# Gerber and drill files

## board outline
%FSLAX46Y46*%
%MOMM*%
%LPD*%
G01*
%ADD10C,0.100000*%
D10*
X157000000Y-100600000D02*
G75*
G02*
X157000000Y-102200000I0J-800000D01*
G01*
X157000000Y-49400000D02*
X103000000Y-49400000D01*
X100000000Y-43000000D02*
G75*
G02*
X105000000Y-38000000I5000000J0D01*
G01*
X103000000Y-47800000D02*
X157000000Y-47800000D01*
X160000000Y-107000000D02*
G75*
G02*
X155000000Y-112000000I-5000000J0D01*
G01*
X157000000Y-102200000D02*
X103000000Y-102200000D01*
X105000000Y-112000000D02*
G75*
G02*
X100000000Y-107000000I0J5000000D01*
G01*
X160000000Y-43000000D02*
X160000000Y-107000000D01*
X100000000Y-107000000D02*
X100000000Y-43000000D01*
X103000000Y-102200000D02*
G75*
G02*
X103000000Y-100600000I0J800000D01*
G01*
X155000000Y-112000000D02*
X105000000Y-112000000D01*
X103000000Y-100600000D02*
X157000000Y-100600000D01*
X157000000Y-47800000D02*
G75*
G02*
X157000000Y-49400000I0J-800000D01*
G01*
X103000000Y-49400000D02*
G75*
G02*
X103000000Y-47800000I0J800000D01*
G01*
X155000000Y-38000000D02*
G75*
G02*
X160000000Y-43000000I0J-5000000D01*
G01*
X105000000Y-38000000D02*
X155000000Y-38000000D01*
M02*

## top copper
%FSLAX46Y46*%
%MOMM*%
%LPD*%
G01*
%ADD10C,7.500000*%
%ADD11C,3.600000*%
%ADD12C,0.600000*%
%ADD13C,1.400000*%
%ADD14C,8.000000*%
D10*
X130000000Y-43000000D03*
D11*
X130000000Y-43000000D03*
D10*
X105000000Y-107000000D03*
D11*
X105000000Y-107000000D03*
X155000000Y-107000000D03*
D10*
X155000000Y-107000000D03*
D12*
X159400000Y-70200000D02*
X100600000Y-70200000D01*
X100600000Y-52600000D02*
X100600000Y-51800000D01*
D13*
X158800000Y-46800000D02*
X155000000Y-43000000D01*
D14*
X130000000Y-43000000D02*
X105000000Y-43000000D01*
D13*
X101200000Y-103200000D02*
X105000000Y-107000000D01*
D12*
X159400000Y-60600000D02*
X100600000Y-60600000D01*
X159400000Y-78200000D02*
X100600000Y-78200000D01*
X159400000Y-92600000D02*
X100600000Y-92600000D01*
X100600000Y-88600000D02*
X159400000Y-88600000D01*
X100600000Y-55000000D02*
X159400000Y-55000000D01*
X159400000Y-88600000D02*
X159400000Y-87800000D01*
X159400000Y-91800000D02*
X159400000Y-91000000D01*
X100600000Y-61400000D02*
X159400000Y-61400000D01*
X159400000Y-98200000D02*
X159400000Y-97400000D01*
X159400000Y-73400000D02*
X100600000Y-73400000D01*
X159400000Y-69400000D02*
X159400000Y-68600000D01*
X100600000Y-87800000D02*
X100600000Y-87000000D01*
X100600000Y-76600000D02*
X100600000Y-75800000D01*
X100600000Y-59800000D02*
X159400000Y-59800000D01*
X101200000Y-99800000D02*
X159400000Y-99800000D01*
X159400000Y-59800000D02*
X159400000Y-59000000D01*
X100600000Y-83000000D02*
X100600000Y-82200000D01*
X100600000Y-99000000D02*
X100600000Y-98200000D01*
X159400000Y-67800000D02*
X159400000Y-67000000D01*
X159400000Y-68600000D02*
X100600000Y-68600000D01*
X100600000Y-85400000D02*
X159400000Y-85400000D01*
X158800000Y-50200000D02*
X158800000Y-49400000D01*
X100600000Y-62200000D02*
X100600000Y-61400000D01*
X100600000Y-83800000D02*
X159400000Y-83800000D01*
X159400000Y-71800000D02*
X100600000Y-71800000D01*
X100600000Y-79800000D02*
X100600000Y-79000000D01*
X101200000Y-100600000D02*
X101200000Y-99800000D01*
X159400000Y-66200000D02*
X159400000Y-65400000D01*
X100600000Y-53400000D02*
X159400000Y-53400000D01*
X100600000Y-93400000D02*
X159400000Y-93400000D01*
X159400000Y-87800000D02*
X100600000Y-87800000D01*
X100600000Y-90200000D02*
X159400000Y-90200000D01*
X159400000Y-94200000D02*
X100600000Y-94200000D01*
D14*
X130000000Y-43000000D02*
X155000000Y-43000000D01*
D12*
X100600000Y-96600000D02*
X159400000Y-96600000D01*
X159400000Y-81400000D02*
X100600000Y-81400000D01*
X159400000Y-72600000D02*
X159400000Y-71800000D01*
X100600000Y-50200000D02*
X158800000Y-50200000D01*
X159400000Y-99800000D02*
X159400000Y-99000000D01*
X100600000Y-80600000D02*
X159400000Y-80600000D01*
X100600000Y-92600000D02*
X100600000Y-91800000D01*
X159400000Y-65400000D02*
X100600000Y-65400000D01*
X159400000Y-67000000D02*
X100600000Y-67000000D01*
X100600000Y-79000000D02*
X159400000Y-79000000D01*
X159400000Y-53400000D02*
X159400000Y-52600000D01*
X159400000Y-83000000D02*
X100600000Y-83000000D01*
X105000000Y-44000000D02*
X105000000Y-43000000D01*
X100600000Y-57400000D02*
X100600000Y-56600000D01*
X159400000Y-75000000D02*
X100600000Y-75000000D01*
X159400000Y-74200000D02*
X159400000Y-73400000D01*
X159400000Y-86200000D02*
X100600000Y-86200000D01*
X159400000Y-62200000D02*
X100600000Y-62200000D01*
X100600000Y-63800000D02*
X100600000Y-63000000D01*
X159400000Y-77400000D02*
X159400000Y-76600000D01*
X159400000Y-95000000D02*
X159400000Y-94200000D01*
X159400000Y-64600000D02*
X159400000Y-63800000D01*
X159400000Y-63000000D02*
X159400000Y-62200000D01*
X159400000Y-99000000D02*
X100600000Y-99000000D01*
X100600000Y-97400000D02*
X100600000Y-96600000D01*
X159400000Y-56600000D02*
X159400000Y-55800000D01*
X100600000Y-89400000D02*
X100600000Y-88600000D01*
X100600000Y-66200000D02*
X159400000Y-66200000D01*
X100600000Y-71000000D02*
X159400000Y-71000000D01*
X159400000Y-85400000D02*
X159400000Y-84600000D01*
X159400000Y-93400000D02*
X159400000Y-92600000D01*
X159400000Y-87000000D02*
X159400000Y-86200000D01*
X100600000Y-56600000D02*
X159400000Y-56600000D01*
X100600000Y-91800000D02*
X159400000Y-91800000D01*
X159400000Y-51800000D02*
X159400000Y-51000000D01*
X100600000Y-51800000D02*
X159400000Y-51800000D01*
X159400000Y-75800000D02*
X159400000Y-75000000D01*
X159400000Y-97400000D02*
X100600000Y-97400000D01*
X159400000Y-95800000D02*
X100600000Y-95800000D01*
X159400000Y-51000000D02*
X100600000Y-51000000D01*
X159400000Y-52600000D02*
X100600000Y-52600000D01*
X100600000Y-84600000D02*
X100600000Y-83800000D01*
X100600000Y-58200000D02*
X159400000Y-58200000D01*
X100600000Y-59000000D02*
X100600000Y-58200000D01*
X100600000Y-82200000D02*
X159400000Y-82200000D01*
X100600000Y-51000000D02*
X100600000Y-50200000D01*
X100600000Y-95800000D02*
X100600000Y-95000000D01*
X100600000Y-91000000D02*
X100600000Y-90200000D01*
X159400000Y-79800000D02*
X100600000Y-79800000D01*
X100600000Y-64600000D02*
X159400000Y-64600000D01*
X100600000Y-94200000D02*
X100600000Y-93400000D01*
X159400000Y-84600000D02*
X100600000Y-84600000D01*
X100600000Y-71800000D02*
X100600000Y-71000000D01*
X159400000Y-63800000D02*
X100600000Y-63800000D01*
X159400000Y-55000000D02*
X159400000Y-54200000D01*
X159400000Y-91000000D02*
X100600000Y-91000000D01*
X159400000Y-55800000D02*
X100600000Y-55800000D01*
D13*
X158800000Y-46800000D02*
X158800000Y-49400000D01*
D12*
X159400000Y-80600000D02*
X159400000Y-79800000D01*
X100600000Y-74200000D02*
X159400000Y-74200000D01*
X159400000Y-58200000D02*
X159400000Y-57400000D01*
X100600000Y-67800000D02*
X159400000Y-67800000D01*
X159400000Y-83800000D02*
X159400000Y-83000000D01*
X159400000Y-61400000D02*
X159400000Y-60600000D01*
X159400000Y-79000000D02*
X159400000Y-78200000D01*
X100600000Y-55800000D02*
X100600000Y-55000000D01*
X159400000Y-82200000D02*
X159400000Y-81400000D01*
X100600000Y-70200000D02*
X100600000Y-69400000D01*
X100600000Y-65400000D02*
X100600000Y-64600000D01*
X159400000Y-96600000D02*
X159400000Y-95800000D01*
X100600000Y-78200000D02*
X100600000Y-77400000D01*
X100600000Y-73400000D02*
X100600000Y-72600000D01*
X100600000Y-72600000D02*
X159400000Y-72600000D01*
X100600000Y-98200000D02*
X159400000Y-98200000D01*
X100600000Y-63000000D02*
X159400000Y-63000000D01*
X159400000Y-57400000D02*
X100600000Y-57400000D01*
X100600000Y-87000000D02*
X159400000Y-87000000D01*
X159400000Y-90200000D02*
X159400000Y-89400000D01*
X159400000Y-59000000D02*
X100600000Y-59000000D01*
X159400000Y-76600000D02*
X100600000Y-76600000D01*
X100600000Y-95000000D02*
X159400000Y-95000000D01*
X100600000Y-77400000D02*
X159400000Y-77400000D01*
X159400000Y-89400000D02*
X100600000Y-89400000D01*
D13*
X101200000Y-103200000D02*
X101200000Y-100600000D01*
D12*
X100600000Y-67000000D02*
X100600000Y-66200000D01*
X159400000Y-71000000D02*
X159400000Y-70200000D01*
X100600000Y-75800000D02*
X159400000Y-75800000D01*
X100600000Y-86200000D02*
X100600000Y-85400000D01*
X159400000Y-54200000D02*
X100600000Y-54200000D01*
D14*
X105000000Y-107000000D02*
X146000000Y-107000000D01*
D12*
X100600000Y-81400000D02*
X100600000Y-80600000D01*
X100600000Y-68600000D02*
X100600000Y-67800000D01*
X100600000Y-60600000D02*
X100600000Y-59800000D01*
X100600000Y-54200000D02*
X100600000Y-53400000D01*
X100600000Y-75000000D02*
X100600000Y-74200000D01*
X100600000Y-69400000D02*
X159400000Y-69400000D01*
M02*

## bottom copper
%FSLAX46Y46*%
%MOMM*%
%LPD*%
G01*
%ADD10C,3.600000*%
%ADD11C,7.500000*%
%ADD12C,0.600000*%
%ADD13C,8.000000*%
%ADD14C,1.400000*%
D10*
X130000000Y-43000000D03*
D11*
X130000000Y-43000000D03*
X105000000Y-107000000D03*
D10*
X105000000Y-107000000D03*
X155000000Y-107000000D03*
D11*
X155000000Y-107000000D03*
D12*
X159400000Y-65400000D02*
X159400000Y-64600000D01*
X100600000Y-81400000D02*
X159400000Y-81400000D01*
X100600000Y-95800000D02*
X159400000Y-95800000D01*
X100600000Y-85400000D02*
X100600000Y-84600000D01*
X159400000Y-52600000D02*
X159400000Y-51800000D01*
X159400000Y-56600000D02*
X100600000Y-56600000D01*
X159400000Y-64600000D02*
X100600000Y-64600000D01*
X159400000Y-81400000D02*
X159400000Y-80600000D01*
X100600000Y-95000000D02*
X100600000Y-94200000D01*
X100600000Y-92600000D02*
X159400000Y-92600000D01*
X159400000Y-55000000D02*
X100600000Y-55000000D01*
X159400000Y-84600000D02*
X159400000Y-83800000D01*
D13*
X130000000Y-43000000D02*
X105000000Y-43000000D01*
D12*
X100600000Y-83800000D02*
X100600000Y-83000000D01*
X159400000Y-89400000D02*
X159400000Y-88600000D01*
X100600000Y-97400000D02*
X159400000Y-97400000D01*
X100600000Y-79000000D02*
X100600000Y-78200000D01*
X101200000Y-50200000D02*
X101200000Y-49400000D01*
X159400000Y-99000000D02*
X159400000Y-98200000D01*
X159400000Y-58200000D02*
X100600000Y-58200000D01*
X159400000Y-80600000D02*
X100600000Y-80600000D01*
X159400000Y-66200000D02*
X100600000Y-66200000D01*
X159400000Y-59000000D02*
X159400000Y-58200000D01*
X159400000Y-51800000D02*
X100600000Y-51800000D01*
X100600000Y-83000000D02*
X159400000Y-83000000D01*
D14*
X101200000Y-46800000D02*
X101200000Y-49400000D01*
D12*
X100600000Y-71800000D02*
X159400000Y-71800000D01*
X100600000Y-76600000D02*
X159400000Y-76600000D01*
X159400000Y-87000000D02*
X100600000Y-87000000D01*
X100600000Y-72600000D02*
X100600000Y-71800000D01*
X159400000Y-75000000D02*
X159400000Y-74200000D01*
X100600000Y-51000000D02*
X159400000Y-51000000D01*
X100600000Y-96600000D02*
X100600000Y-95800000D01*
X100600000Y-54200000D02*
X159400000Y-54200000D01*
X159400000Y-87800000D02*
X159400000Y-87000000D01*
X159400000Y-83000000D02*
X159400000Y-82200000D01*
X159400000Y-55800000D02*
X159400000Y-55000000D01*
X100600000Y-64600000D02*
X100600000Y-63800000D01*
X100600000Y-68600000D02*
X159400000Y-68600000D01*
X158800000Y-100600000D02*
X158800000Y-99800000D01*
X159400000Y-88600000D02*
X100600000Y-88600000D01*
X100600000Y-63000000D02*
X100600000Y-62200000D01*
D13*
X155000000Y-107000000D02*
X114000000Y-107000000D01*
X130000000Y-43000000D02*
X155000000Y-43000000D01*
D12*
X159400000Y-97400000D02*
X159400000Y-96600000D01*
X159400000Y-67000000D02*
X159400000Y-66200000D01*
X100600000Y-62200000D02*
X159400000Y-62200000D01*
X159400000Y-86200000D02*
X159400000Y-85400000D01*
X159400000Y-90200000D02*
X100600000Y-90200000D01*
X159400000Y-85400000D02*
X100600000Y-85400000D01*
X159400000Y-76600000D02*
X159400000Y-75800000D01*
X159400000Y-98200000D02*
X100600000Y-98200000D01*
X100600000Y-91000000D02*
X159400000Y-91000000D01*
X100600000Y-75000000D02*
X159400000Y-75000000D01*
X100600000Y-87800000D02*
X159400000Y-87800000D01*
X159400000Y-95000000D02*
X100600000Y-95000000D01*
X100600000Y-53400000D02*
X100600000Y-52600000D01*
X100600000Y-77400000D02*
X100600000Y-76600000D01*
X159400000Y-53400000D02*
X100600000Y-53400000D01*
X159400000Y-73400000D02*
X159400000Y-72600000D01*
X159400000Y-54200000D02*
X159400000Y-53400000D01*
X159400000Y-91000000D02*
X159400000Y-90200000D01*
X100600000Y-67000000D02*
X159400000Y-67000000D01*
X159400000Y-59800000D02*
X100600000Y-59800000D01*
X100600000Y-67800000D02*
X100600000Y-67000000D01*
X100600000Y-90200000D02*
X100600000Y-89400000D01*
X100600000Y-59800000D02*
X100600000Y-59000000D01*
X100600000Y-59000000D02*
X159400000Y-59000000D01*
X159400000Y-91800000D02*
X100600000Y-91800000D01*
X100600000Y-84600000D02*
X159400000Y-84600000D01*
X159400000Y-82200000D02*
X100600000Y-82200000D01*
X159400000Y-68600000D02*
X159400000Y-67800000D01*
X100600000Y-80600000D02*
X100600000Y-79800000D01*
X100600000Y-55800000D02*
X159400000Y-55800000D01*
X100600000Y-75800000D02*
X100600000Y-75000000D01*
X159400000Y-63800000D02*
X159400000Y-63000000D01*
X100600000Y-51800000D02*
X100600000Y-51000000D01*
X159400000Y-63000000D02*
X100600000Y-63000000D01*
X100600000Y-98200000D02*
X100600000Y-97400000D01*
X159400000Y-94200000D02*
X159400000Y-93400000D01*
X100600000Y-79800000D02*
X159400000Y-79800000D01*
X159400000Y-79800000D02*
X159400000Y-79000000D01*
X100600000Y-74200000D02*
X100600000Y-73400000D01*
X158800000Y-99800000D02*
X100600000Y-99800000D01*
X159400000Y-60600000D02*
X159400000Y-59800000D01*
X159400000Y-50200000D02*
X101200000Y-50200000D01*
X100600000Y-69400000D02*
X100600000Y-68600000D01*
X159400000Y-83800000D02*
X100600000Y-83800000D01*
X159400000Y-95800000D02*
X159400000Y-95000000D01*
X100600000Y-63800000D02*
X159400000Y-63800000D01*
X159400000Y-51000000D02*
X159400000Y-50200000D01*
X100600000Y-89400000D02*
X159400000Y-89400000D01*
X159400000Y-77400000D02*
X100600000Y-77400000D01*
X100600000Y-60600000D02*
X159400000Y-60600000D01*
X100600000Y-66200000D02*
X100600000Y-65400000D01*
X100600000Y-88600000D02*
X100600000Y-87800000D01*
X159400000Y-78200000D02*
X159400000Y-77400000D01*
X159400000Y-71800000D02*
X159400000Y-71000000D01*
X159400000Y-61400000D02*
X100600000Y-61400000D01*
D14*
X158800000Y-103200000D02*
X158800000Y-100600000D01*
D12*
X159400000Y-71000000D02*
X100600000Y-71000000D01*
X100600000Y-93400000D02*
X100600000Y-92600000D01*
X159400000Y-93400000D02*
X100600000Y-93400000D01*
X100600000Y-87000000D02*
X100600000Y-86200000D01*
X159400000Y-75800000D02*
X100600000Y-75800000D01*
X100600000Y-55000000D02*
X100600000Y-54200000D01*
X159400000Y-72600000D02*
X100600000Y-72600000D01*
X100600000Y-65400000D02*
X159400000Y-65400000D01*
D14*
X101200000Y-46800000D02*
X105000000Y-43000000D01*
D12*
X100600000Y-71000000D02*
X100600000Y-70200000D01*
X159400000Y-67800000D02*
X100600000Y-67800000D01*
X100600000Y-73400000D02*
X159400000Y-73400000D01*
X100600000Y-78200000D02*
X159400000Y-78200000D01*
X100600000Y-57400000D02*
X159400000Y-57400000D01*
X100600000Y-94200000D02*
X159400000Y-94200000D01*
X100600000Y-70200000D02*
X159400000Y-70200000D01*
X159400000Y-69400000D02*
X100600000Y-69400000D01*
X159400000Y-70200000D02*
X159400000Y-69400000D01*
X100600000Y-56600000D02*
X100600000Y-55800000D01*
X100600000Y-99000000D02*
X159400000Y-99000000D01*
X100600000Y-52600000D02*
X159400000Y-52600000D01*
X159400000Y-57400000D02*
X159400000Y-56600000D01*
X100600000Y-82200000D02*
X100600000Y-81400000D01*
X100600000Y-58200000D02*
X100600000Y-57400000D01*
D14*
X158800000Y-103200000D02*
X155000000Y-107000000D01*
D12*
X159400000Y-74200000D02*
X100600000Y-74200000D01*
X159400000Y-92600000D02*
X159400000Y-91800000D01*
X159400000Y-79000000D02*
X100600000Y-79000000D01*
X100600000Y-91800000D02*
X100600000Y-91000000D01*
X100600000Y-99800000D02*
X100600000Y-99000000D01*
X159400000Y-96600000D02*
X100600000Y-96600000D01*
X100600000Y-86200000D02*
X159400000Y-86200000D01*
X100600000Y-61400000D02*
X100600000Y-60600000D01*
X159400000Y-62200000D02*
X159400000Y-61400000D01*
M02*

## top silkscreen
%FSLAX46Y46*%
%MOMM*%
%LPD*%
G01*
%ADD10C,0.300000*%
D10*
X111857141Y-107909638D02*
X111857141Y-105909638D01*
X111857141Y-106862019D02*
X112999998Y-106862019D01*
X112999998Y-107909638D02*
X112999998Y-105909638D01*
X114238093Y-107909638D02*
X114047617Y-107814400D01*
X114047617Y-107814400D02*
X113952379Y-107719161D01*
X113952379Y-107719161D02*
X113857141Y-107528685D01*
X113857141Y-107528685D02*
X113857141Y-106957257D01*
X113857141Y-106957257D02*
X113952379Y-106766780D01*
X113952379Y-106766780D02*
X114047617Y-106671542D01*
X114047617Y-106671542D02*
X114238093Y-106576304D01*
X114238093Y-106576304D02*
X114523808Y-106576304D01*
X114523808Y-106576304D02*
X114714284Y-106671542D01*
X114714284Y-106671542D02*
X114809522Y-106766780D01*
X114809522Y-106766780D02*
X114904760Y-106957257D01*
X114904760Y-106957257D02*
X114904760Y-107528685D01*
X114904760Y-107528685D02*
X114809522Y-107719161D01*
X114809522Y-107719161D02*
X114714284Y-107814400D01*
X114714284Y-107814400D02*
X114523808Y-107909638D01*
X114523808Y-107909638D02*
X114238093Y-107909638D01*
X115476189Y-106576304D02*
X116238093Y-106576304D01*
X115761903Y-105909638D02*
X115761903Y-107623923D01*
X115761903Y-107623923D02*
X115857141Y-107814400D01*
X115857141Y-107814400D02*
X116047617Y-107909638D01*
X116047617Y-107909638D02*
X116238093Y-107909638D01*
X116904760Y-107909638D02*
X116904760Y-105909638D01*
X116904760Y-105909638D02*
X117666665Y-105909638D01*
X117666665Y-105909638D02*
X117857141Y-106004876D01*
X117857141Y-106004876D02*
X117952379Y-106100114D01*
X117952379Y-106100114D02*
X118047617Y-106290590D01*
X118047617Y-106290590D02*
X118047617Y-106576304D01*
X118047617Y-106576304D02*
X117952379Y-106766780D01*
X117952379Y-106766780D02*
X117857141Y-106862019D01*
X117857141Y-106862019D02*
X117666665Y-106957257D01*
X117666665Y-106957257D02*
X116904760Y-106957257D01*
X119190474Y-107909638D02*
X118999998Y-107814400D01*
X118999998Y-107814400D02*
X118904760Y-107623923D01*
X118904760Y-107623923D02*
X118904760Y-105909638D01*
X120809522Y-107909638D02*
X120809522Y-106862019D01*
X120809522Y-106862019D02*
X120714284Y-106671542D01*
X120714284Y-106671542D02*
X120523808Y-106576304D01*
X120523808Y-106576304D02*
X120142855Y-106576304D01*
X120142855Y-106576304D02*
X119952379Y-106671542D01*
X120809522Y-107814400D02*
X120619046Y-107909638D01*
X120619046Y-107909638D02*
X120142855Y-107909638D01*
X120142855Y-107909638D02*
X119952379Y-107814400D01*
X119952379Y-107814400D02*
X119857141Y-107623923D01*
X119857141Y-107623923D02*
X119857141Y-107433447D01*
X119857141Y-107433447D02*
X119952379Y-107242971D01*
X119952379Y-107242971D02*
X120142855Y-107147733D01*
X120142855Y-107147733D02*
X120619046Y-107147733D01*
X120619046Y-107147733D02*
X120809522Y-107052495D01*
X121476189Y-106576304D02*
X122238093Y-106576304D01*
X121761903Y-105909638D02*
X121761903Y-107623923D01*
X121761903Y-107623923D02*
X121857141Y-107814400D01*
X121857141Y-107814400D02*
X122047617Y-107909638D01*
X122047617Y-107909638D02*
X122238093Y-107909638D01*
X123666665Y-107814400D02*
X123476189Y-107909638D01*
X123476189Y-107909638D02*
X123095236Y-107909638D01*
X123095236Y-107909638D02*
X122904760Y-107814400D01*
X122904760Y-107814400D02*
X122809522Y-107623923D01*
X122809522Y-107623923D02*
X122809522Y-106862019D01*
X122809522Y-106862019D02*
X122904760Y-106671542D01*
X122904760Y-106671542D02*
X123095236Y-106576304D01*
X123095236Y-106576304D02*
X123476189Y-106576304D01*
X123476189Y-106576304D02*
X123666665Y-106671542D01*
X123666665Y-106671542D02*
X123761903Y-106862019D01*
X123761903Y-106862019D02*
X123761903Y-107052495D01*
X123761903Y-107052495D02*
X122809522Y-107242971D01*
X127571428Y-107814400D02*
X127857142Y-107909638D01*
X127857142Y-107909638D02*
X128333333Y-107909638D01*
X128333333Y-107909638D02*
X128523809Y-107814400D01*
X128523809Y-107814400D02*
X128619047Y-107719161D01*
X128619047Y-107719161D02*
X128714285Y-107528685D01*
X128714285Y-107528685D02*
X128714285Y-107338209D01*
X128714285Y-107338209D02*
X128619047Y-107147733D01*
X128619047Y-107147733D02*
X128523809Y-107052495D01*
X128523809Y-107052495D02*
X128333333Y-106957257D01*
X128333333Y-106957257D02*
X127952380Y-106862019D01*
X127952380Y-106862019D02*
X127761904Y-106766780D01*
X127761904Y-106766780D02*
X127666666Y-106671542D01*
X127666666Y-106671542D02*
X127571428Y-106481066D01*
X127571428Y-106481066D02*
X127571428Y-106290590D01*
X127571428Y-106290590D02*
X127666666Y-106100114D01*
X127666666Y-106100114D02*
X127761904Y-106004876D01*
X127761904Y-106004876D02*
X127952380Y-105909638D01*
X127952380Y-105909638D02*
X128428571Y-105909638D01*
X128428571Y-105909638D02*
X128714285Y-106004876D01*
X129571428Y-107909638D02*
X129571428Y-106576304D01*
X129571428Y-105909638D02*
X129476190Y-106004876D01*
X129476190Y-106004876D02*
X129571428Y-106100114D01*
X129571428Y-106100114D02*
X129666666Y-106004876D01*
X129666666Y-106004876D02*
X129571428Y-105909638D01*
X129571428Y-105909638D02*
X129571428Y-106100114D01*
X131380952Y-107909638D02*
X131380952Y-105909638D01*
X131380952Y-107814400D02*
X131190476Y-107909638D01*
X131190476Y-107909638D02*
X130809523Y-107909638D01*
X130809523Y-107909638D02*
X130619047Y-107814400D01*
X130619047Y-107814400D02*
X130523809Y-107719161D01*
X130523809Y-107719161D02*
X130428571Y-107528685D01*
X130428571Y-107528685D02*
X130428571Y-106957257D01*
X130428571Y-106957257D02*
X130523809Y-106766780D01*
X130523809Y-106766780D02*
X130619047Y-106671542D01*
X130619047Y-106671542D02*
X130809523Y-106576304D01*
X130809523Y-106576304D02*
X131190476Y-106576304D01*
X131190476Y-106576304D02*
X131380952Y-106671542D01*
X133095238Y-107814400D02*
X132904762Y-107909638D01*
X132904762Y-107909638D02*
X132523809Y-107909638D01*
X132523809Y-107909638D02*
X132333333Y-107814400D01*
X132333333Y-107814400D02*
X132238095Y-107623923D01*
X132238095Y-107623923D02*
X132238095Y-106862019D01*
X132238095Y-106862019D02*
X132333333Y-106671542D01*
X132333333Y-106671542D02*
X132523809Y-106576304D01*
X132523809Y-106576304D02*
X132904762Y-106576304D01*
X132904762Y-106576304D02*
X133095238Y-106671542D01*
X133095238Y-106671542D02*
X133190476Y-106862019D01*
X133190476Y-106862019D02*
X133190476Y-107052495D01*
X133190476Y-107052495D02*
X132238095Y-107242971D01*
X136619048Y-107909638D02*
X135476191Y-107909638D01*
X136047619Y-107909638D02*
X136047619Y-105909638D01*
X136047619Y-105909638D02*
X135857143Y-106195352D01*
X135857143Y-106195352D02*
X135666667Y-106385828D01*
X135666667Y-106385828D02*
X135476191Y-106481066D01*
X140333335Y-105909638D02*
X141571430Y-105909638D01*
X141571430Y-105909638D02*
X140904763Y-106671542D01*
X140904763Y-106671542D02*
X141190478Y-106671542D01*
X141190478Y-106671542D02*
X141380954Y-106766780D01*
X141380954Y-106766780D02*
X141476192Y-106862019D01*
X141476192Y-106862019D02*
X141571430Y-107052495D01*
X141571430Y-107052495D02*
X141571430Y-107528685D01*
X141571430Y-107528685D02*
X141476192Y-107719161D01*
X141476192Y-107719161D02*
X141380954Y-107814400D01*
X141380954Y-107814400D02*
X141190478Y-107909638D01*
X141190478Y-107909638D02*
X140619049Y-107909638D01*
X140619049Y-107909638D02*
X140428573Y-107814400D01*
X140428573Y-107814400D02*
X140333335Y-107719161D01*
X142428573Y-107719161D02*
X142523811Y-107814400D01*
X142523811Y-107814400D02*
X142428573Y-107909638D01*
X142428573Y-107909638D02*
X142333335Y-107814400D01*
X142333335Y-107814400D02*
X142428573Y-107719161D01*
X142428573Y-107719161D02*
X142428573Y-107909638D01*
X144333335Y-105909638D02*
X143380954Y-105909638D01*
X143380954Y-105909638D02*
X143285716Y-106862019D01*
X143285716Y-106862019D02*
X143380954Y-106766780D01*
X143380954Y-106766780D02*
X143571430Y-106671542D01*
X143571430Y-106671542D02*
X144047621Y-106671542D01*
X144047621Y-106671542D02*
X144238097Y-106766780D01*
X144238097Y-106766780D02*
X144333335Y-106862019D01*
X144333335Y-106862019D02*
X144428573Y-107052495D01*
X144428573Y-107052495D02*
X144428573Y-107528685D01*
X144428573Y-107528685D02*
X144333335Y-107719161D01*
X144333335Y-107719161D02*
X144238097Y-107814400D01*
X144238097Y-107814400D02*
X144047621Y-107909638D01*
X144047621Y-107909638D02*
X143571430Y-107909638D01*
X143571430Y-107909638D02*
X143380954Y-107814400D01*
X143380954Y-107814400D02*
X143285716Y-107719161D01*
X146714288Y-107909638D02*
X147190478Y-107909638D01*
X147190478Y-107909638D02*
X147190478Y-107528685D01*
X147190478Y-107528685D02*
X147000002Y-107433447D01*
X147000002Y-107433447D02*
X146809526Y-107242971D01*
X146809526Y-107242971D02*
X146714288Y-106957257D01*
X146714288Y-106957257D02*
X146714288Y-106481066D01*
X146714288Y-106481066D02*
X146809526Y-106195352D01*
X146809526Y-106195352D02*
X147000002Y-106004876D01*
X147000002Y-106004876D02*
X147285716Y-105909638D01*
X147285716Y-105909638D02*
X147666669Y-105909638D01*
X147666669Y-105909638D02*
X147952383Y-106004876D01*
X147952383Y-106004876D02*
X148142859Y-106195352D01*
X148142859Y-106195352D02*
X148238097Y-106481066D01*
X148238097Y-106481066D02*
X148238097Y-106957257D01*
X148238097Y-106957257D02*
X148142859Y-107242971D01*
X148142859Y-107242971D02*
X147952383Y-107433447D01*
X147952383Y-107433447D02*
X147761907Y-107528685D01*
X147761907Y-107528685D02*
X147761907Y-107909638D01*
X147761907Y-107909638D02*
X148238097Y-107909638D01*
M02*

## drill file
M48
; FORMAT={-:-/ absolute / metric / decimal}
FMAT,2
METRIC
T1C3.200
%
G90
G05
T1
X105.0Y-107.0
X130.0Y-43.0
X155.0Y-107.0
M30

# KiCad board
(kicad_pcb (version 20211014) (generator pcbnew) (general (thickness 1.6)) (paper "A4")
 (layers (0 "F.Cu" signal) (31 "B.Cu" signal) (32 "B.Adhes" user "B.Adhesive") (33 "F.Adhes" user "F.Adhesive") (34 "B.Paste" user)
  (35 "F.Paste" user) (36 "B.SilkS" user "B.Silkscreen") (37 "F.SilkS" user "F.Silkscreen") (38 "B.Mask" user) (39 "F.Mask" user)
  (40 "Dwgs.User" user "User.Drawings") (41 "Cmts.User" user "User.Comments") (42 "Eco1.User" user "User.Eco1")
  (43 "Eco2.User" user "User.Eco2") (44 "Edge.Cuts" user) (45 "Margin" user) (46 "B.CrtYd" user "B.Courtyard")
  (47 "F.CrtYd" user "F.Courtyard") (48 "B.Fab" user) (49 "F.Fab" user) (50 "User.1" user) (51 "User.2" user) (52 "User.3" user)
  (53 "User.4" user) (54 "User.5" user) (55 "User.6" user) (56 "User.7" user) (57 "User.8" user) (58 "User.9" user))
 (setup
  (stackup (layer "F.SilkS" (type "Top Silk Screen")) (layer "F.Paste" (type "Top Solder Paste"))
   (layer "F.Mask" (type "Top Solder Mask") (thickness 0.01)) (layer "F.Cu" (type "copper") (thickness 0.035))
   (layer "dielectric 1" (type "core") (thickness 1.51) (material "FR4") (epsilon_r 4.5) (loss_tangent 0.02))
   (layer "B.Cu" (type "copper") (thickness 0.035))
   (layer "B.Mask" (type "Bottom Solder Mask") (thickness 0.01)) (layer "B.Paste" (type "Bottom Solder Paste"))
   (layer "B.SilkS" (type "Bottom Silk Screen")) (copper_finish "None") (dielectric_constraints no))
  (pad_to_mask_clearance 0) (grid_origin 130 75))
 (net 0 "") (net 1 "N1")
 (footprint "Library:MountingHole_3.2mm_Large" (layer "F.Cu") (at 130 43)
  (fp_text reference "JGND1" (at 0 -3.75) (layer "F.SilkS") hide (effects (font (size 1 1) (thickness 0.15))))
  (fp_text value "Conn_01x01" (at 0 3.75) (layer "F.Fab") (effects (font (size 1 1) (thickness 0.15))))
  (pad "1" connect circle (at 0 0) (size 7.5 7.5) (layers "F.Cu" "F.Mask") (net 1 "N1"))
  (pad "1" thru_hole circle (at 0 0) (size 3.6 3.6) (drill 3.2) (layers *.Cu *.Mask) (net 1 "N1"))
  (pad "1" connect circle (at 0 0) (size 7.5 7.5) (layers "B.Cu" "B.Mask") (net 1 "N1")))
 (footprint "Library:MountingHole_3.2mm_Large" (layer "F.Cu") (at 105 107)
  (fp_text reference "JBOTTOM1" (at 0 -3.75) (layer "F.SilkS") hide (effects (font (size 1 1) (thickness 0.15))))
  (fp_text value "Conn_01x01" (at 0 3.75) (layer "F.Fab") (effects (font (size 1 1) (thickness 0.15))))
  (pad "1" connect circle (at 0 0) (size 7.5 7.5) (layers "F.Cu" "F.Mask") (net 1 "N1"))
  (pad "1" connect circle (at 0 0) (size 7.5 7.5) (layers "B.Cu" "B.Mask") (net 1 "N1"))
  (pad "1" thru_hole circle (at 0 0) (size 3.6 3.6) (drill 3.2) (layers *.Cu *.Mask) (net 1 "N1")))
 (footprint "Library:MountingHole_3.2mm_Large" (layer "F.Cu") (at 155 107)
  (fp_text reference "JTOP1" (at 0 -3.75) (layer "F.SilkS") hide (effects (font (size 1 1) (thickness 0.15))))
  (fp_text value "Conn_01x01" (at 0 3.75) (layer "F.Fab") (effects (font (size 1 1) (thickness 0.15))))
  (pad "1" thru_hole circle (at 0 0) (size 3.6 3.6) (drill 3.2) (layers *.Cu *.Mask) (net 1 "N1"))
  (pad "1" connect circle (at 0 0) (size 7.5 7.5) (layers "F.Cu" "F.Mask") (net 1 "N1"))
  (pad "1" connect circle (at 0 0) (size 7.5 7.5) (layers "B.Cu" "B.Mask") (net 1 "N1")))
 (gr_arc (start 157 100.6) (mid 157.8 101.4) (end 157 102.2) (layer "Edge.Cuts") (width 0.1))
 (gr_line (start 157 49.4) (end 103 49.4) (layer "Edge.Cuts") (width 0.1))
 (gr_arc (start 100 43) (mid 101.464466 39.464466) (end 105 38) (layer "Edge.Cuts") (width 0.1))
 (gr_line (start 103 47.8) (end 157 47.8) (layer "Edge.Cuts") (width 0.1))
 (gr_arc (start 160 107) (mid 158.535534 110.535534) (end 155 112) (layer "Edge.Cuts") (width 0.1))
 (gr_line (start 157 102.2) (end 103 102.2) (layer "Edge.Cuts") (width 0.1))
 (gr_arc (start 105 112) (mid 101.464466 110.535534) (end 100 107) (layer "Edge.Cuts") (width 0.1))
 (gr_line (start 160 43) (end 160 107) (layer "Edge.Cuts") (width 0.1))
 (gr_line (start 100 107) (end 100 43) (layer "Edge.Cuts") (width 0.1))
 (gr_arc (start 103 102.2) (mid 102.2 101.4) (end 103 100.6) (layer "Edge.Cuts") (width 0.1))
 (gr_line (start 155 112) (end 105 112) (layer "Edge.Cuts") (width 0.1))
 (gr_line (start 103 100.6) (end 157 100.6) (layer "Edge.Cuts") (width 0.1))
 (gr_arc (start 157 47.8) (mid 157.8 48.6) (end 157 49.4) (layer "Edge.Cuts") (width 0.1))
 (gr_arc (start 103 49.4) (mid 102.2 48.6) (end 103 47.8) (layer "Edge.Cuts") (width 0.1))
 (gr_arc (start 155 38) (mid 158.535534 39.464466) (end 160 43) (layer "Edge.Cuts") (width 0.1))
 (gr_line (start 105 38) (end 155 38) (layer "Edge.Cuts") (width 0.1))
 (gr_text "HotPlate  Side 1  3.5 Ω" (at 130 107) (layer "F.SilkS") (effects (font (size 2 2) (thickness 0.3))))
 (segment (start 159.4 70.2) (end 100.6 70.2) (width 0.6) (layer "F.Cu") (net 1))
 (segment (start 100.6 52.6) (end 100.6 51.8) (width 0.6) (layer "F.Cu") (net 1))
 (segment (start 158.8 46.8) (end 155 43) (width 1.4) (layer "F.Cu") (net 1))
 (segment (start 130 43) (end 105 43) (width 8) (layer "F.Cu") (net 1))
 (segment (start 101.2 103.2) (end 105 107) (width 1.4) (layer "F.Cu") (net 1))
 (segment (start 159.4 60.6) (end 100.6 60.6) (width 0.6) (layer "F.Cu") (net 1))
 (segment (start 159.4 78.2) (end 100.6 78.2) (width 0.6) (layer "F.Cu") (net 1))
 (segment (start 159.4 92.6) (end 100.6 92.6) (width 0.6) (layer "F.Cu") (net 1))
 (segment (start 100.6 88.6) (end 159.4 88.6) (width 0.6) (layer "F.Cu") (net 1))
 (segment (start 100.6 55) (end 159.4 55) (width 0.6) (layer "F.Cu") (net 1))
 (segment (start 159.4 88.6) (end 159.4 87.8) (width 0.6) (layer "F.Cu") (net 1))
 (segment (start 159.4 91.8) (end 159.4 91) (width 0.6) (layer "F.Cu") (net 1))
 (segment (start 100.6 61.4) (end 159.4 61.4) (width 0.6) (layer "F.Cu") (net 1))
 (segment (start 159.4 98.2) (end 159.4 97.4) (width 0.6) (layer "F.Cu") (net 1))
 (segment (start 159.4 73.4) (end 100.6 73.4) (width 0.6) (layer "F.Cu") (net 1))
 (segment (start 159.4 69.4) (end 159.4 68.6) (width 0.6) (layer "F.Cu") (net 1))
 (segment (start 100.6 87.8) (end 100.6 87) (width 0.6) (layer "F.Cu") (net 1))
 (segment (start 100.6 76.6) (end 100.6 75.8) (width 0.6) (layer "F.Cu") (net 1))
 (segment (start 100.6 59.8) (end 159.4 59.8) (width 0.6) (layer "F.Cu") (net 1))
 (segment (start 101.2 99.8) (end 159.4 99.8) (width 0.6) (layer "F.Cu") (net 1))
 (segment (start 159.4 59.8) (end 159.4 59) (width 0.6) (layer "F.Cu") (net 1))
 (segment (start 100.6 83) (end 100.6 82.2) (width 0.6) (layer "F.Cu") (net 1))
 (segment (start 100.6 99) (end 100.6 98.2) (width 0.6) (layer "F.Cu") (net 1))
 (segment (start 159.4 67.8) (end 159.4 67) (width 0.6) (layer "F.Cu") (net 1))
 (segment (start 159.4 68.6) (end 100.6 68.6) (width 0.6) (layer "F.Cu") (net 1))
 (segment (start 100.6 85.4) (end 159.4 85.4) (width 0.6) (layer "F.Cu") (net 1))
 (segment (start 158.8 50.2) (end 158.8 49.4) (width 0.6) (layer "F.Cu") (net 1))
 (segment (start 100.6 62.2) (end 100.6 61.4) (width 0.6) (layer "F.Cu") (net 1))
 (segment (start 100.6 83.8) (end 159.4 83.8) (width 0.6) (layer "F.Cu") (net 1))
 (segment (start 159.4 71.8) (end 100.6 71.8) (width 0.6) (layer "F.Cu") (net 1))
 (segment (start 100.6 79.8) (end 100.6 79) (width 0.6) (layer "F.Cu") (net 1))
 (segment (start 101.2 100.6) (end 101.2 99.8) (width 0.6) (layer "F.Cu") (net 1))
 (segment (start 159.4 66.2) (end 159.4 65.4) (width 0.6) (layer "F.Cu") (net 1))
 (segment (start 100.6 53.4) (end 159.4 53.4) (width 0.6) (layer "F.Cu") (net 1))
 (segment (start 100.6 93.4) (end 159.4 93.4) (width 0.6) (layer "F.Cu") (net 1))
 (segment (start 159.4 87.8) (end 100.6 87.8) (width 0.6) (layer "F.Cu") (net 1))
 (segment (start 100.6 90.2) (end 159.4 90.2) (width 0.6) (layer "F.Cu") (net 1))
 (segment (start 159.4 94.2) (end 100.6 94.2) (width 0.6) (layer "F.Cu") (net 1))
 (segment (start 130 43) (end 155 43) (width 8) (layer "F.Cu") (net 1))
 (segment (start 100.6 96.6) (end 159.4 96.6) (width 0.6) (layer "F.Cu") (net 1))
 (segment (start 159.4 81.4) (end 100.6 81.4) (width 0.6) (layer "F.Cu") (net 1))
 (segment (start 159.4 72.6) (end 159.4 71.8) (width 0.6) (layer "F.Cu") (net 1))
 (segment (start 100.6 50.2) (end 158.8 50.2) (width 0.6) (layer "F.Cu") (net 1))
 (segment (start 159.4 99.8) (end 159.4 99) (width 0.6) (layer "F.Cu") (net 1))
 (segment (start 100.6 80.6) (end 159.4 80.6) (width 0.6) (layer "F.Cu") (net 1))
 (segment (start 100.6 92.6) (end 100.6 91.8) (width 0.6) (layer "F.Cu") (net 1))
 (segment (start 159.4 65.4) (end 100.6 65.4) (width 0.6) (layer "F.Cu") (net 1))
 (segment (start 159.4 67) (end 100.6 67) (width 0.6) (layer "F.Cu") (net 1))
 (segment (start 100.6 79) (end 159.4 79) (width 0.6) (layer "F.Cu") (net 1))
 (segment (start 159.4 53.4) (end 159.4 52.6) (width 0.6) (layer "F.Cu") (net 1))
 (segment (start 159.4 83) (end 100.6 83) (width 0.6) (layer "F.Cu") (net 1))
 (segment (start 105 44) (end 105 43) (width 0.6) (layer "F.Cu") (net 1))
 (segment (start 100.6 57.4) (end 100.6 56.6) (width 0.6) (layer "F.Cu") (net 1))
 (segment (start 159.4 75) (end 100.6 75) (width 0.6) (layer "F.Cu") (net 1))
 (segment (start 159.4 74.2) (end 159.4 73.4) (width 0.6) (layer "F.Cu") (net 1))
 (segment (start 159.4 86.2) (end 100.6 86.2) (width 0.6) (layer "F.Cu") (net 1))
 (segment (start 159.4 62.2) (end 100.6 62.2) (width 0.6) (layer "F.Cu") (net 1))
 (segment (start 100.6 63.8) (end 100.6 63) (width 0.6) (layer "F.Cu") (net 1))
 (segment (start 159.4 77.4) (end 159.4 76.6) (width 0.6) (layer "F.Cu") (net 1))
 (segment (start 159.4 95) (end 159.4 94.2) (width 0.6) (layer "F.Cu") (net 1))
 (segment (start 159.4 64.6) (end 159.4 63.8) (width 0.6) (layer "F.Cu") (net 1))
 (segment (start 159.4 63) (end 159.4 62.2) (width 0.6) (layer "F.Cu") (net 1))
 (segment (start 159.4 99) (end 100.6 99) (width 0.6) (layer "F.Cu") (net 1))
 (segment (start 100.6 97.4) (end 100.6 96.6) (width 0.6) (layer "F.Cu") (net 1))
 (segment (start 159.4 56.6) (end 159.4 55.8) (width 0.6) (layer "F.Cu") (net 1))
 (segment (start 100.6 89.4) (end 100.6 88.6) (width 0.6) (layer "F.Cu") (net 1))
 (segment (start 100.6 66.2) (end 159.4 66.2) (width 0.6) (layer "F.Cu") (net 1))
 (segment (start 100.6 71) (end 159.4 71) (width 0.6) (layer "F.Cu") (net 1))
 (segment (start 159.4 85.4) (end 159.4 84.6) (width 0.6) (layer "F.Cu") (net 1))
 (segment (start 159.4 93.4) (end 159.4 92.6) (width 0.6) (layer "F.Cu") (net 1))
 (segment (start 159.4 87) (end 159.4 86.2) (width 0.6) (layer "F.Cu") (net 1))
 (segment (start 100.6 56.6) (end 159.4 56.6) (width 0.6) (layer "F.Cu") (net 1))
 (segment (start 100.6 91.8) (end 159.4 91.8) (width 0.6) (layer "F.Cu") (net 1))
 (segment (start 159.4 51.8) (end 159.4 51) (width 0.6) (layer "F.Cu") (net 1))
 (segment (start 100.6 51.8) (end 159.4 51.8) (width 0.6) (layer "F.Cu") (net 1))
 (segment (start 159.4 75.8) (end 159.4 75) (width 0.6) (layer "F.Cu") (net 1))
 (segment (start 159.4 97.4) (end 100.6 97.4) (width 0.6) (layer "F.Cu") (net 1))
 (segment (start 159.4 95.8) (end 100.6 95.8) (width 0.6) (layer "F.Cu") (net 1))
 (segment (start 159.4 51) (end 100.6 51) (width 0.6) (layer "F.Cu") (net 1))
 (segment (start 159.4 52.6) (end 100.6 52.6) (width 0.6) (layer "F.Cu") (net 1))
 (segment (start 100.6 84.6) (end 100.6 83.8) (width 0.6) (layer "F.Cu") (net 1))
 (segment (start 100.6 58.2) (end 159.4 58.2) (width 0.6) (layer "F.Cu") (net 1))
 (segment (start 100.6 59) (end 100.6 58.2) (width 0.6) (layer "F.Cu") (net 1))
 (segment (start 100.6 82.2) (end 159.4 82.2) (width 0.6) (layer "F.Cu") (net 1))
 (segment (start 100.6 51) (end 100.6 50.2) (width 0.6) (layer "F.Cu") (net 1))
 (segment (start 100.6 95.8) (end 100.6 95) (width 0.6) (layer "F.Cu") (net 1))
 (segment (start 100.6 91) (end 100.6 90.2) (width 0.6) (layer "F.Cu") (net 1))
 (segment (start 159.4 79.8) (end 100.6 79.8) (width 0.6) (layer "F.Cu") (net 1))
 (segment (start 100.6 64.6) (end 159.4 64.6) (width 0.6) (layer "F.Cu") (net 1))
 (segment (start 100.6 94.2) (end 100.6 93.4) (width 0.6) (layer "F.Cu") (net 1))
 (segment (start 159.4 84.6) (end 100.6 84.6) (width 0.6) (layer "F.Cu") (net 1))
 (segment (start 100.6 71.8) (end 100.6 71) (width 0.6) (layer "F.Cu") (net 1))
 (segment (start 159.4 63.8) (end 100.6 63.8) (width 0.6) (layer "F.Cu") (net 1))
 (segment (start 159.4 55) (end 159.4 54.2) (width 0.6) (layer "F.Cu") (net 1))
 (segment (start 159.4 91) (end 100.6 91) (width 0.6) (layer "F.Cu") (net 1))
 (segment (start 159.4 55.8) (end 100.6 55.8) (width 0.6) (layer "F.Cu") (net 1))
 (segment (start 158.8 46.8) (end 158.8 49.4) (width 1.4) (layer "F.Cu") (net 1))
 (segment (start 159.4 80.6) (end 159.4 79.8) (width 0.6) (layer "F.Cu") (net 1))
 (segment (start 100.6 74.2) (end 159.4 74.2) (width 0.6) (layer "F.Cu") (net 1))
 (segment (start 159.4 58.2) (end 159.4 57.4) (width 0.6) (layer "F.Cu") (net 1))
 (segment (start 100.6 67.8) (end 159.4 67.8) (width 0.6) (layer "F.Cu") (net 1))
 (segment (start 159.4 83.8) (end 159.4 83) (width 0.6) (layer "F.Cu") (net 1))
 (segment (start 159.4 61.4) (end 159.4 60.6) (width 0.6) (layer "F.Cu") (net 1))
 (segment (start 159.4 79) (end 159.4 78.2) (width 0.6) (layer "F.Cu") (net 1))
 (segment (start 100.6 55.8) (end 100.6 55) (width 0.6) (layer "F.Cu") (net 1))
 (segment (start 159.4 82.2) (end 159.4 81.4) (width 0.6) (layer "F.Cu") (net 1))
 (segment (start 100.6 70.2) (end 100.6 69.4) (width 0.6) (layer "F.Cu") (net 1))
 (segment (start 100.6 65.4) (end 100.6 64.6) (width 0.6) (layer "F.Cu") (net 1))
 (segment (start 159.4 96.6) (end 159.4 95.8) (width 0.6) (layer "F.Cu") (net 1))
 (segment (start 100.6 78.2) (end 100.6 77.4) (width 0.6) (layer "F.Cu") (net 1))
 (segment (start 100.6 73.4) (end 100.6 72.6) (width 0.6) (layer "F.Cu") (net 1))
 (segment (start 100.6 72.6) (end 159.4 72.6) (width 0.6) (layer "F.Cu") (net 1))
 (segment (start 100.6 98.2) (end 159.4 98.2) (width 0.6) (layer "F.Cu") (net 1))
 (segment (start 100.6 63) (end 159.4 63) (width 0.6) (layer "F.Cu") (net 1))
 (segment (start 159.4 57.4) (end 100.6 57.4) (width 0.6) (layer "F.Cu") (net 1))
 (segment (start 100.6 87) (end 159.4 87) (width 0.6) (layer "F.Cu") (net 1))
 (segment (start 159.4 90.2) (end 159.4 89.4) (width 0.6) (layer "F.Cu") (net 1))
 (segment (start 159.4 59) (end 100.6 59) (width 0.6) (layer "F.Cu") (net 1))
 (segment (start 159.4 76.6) (end 100.6 76.6) (width 0.6) (layer "F.Cu") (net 1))
 (segment (start 100.6 95) (end 159.4 95) (width 0.6) (layer "F.Cu") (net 1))
 (segment (start 100.6 77.4) (end 159.4 77.4) (width 0.6) (layer "F.Cu") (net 1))
 (segment (start 159.4 89.4) (end 100.6 89.4) (width 0.6) (layer "F.Cu") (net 1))
 (segment (start 101.2 103.2) (end 101.2 100.6) (width 1.4) (layer "F.Cu") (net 1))
 (segment (start 100.6 67) (end 100.6 66.2) (width 0.6) (layer "F.Cu") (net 1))
 (segment (start 159.4 71) (end 159.4 70.2) (width 0.6) (layer "F.Cu") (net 1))
 (segment (start 100.6 75.8) (end 159.4 75.8) (width 0.6) (layer "F.Cu") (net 1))
 (segment (start 100.6 86.2) (end 100.6 85.4) (width 0.6) (layer "F.Cu") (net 1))
 (segment (start 159.4 54.2) (end 100.6 54.2) (width 0.6) (layer "F.Cu") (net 1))
 (segment (start 105 107) (end 146 107) (width 8) (layer "F.Cu") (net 1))
 (segment (start 100.6 81.4) (end 100.6 80.6) (width 0.6) (layer "F.Cu") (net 1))
 (segment (start 100.6 68.6) (end 100.6 67.8) (width 0.6) (layer "F.Cu") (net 1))
 (segment (start 100.6 60.6) (end 100.6 59.8) (width 0.6) (layer "F.Cu") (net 1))
 (segment (start 100.6 54.2) (end 100.6 53.4) (width 0.6) (layer "F.Cu") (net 1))
 (segment (start 100.6 75) (end 100.6 74.2) (width 0.6) (layer "F.Cu") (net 1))
 (segment (start 100.6 69.4) (end 159.4 69.4) (width 0.6) (layer "F.Cu") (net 1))
 (segment (start 159.4 65.4) (end 159.4 64.6) (width 0.6) (layer "B.Cu") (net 1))
 (segment (start 100.6 81.4) (end 159.4 81.4) (width 0.6) (layer "B.Cu") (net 1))
 (segment (start 100.6 95.8) (end 159.4 95.8) (width 0.6) (layer "B.Cu") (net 1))
 (segment (start 100.6 85.4) (end 100.6 84.6) (width 0.6) (layer "B.Cu") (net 1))
 (segment (start 159.4 52.6) (end 159.4 51.8) (width 0.6) (layer "B.Cu") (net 1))
 (segment (start 159.4 56.6) (end 100.6 56.6) (width 0.6) (layer "B.Cu") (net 1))
 (segment (start 159.4 64.6) (end 100.6 64.6) (width 0.6) (layer "B.Cu") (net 1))
 (segment (start 159.4 81.4) (end 159.4 80.6) (width 0.6) (layer "B.Cu") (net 1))
 (segment (start 100.6 95) (end 100.6 94.2) (width 0.6) (layer "B.Cu") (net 1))
 (segment (start 100.6 92.6) (end 159.4 92.6) (width 0.6) (layer "B.Cu") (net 1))
 (segment (start 159.4 55) (end 100.6 55) (width 0.6) (layer "B.Cu") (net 1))
 (segment (start 159.4 84.6) (end 159.4 83.8) (width 0.6) (layer "B.Cu") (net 1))
 (segment (start 130 43) (end 105 43) (width 8) (layer "B.Cu") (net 1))
 (segment (start 100.6 83.8) (end 100.6 83) (width 0.6) (layer "B.Cu") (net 1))
 (segment (start 159.4 89.4) (end 159.4 88.6) (width 0.6) (layer "B.Cu") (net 1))
 (segment (start 100.6 97.4) (end 159.4 97.4) (width 0.6) (layer "B.Cu") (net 1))
 (segment (start 100.6 79) (end 100.6 78.2) (width 0.6) (layer "B.Cu") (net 1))
 (segment (start 101.2 50.2) (end 101.2 49.4) (width 0.6) (layer "B.Cu") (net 1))
 (segment (start 159.4 99) (end 159.4 98.2) (width 0.6) (layer "B.Cu") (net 1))
 (segment (start 159.4 58.2) (end 100.6 58.2) (width 0.6) (layer "B.Cu") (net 1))
 (segment (start 159.4 80.6) (end 100.6 80.6) (width 0.6) (layer "B.Cu") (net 1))
 (segment (start 159.4 66.2) (end 100.6 66.2) (width 0.6) (layer "B.Cu") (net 1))
 (segment (start 159.4 59) (end 159.4 58.2) (width 0.6) (layer "B.Cu") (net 1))
 (segment (start 159.4 51.8) (end 100.6 51.8) (width 0.6) (layer "B.Cu") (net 1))
 (segment (start 100.6 83) (end 159.4 83) (width 0.6) (layer "B.Cu") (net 1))
 (segment (start 101.2 46.8) (end 101.2 49.4) (width 1.4) (layer "B.Cu") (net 1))
 (segment (start 100.6 71.8) (end 159.4 71.8) (width 0.6) (layer "B.Cu") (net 1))
 (segment (start 100.6 76.6) (end 159.4 76.6) (width 0.6) (layer "B.Cu") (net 1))
 (segment (start 159.4 87) (end 100.6 87) (width 0.6) (layer "B.Cu") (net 1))
 (segment (start 100.6 72.6) (end 100.6 71.8) (width 0.6) (layer "B.Cu") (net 1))
 (segment (start 159.4 75) (end 159.4 74.2) (width 0.6) (layer "B.Cu") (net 1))
 (segment (start 100.6 51) (end 159.4 51) (width 0.6) (layer "B.Cu") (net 1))
 (segment (start 100.6 96.6) (end 100.6 95.8) (width 0.6) (layer "B.Cu") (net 1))
 (segment (start 100.6 54.2) (end 159.4 54.2) (width 0.6) (layer "B.Cu") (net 1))
 (segment (start 159.4 87.8) (end 159.4 87) (width 0.6) (layer "B.Cu") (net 1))
 (segment (start 159.4 83) (end 159.4 82.2) (width 0.6) (layer "B.Cu") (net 1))
 (segment (start 159.4 55.8) (end 159.4 55) (width 0.6) (layer "B.Cu") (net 1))
 (segment (start 100.6 64.6) (end 100.6 63.8) (width 0.6) (layer "B.Cu") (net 1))
 (segment (start 100.6 68.6) (end 159.4 68.6) (width 0.6) (layer "B.Cu") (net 1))
 (segment (start 158.8 100.6) (end 158.8 99.8) (width 0.6) (layer "B.Cu") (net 1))
 (segment (start 159.4 88.6) (end 100.6 88.6) (width 0.6) (layer "B.Cu") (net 1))
 (segment (start 100.6 63) (end 100.6 62.2) (width 0.6) (layer "B.Cu") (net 1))
 (segment (start 155 107) (end 114 107) (width 8) (layer "B.Cu") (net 1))
 (segment (start 130 43) (end 155 43) (width 8) (layer "B.Cu") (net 1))
 (segment (start 159.4 97.4) (end 159.4 96.6) (width 0.6) (layer "B.Cu") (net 1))
 (segment (start 159.4 67) (end 159.4 66.2) (width 0.6) (layer "B.Cu") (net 1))
 (segment (start 100.6 62.2) (end 159.4 62.2) (width 0.6) (layer "B.Cu") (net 1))
 (segment (start 159.4 86.2) (end 159.4 85.4) (width 0.6) (layer "B.Cu") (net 1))
 (segment (start 159.4 90.2) (end 100.6 90.2) (width 0.6) (layer "B.Cu") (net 1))
 (segment (start 159.4 85.4) (end 100.6 85.4) (width 0.6) (layer "B.Cu") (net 1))
 (segment (start 159.4 76.6) (end 159.4 75.8) (width 0.6) (layer "B.Cu") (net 1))
 (segment (start 159.4 98.2) (end 100.6 98.2) (width 0.6) (layer "B.Cu") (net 1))
 (segment (start 100.6 91) (end 159.4 91) (width 0.6) (layer "B.Cu") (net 1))
 (segment (start 100.6 75) (end 159.4 75) (width 0.6) (layer "B.Cu") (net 1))
 (segment (start 100.6 87.8) (end 159.4 87.8) (width 0.6) (layer "B.Cu") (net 1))
 (segment (start 159.4 95) (end 100.6 95) (width 0.6) (layer "B.Cu") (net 1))
 (segment (start 100.6 53.4) (end 100.6 52.6) (width 0.6) (layer "B.Cu") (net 1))
 (segment (start 100.6 77.4) (end 100.6 76.6) (width 0.6) (layer "B.Cu") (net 1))
 (segment (start 159.4 53.4) (end 100.6 53.4) (width 0.6) (layer "B.Cu") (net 1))
 (segment (start 159.4 73.4) (end 159.4 72.6) (width 0.6) (layer "B.Cu") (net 1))
 (segment (start 159.4 54.2) (end 159.4 53.4) (width 0.6) (layer "B.Cu") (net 1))
 (segment (start 159.4 91) (end 159.4 90.2) (width 0.6) (layer "B.Cu") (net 1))
 (segment (start 100.6 67) (end 159.4 67) (width 0.6) (layer "B.Cu") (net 1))
 (segment (start 159.4 59.8) (end 100.6 59.8) (width 0.6) (layer "B.Cu") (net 1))
 (segment (start 100.6 67.8) (end 100.6 67) (width 0.6) (layer "B.Cu") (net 1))
 (segment (start 100.6 90.2) (end 100.6 89.4) (width 0.6) (layer "B.Cu") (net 1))
 (segment (start 100.6 59.8) (end 100.6 59) (width 0.6) (layer "B.Cu") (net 1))
 (segment (start 100.6 59) (end 159.4 59) (width 0.6) (layer "B.Cu") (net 1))
 (segment (start 159.4 91.8) (end 100.6 91.8) (width 0.6) (layer "B.Cu") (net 1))
 (segment (start 100.6 84.6) (end 159.4 84.6) (width 0.6) (layer "B.Cu") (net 1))
 (segment (start 159.4 82.2) (end 100.6 82.2) (width 0.6) (layer "B.Cu") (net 1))
 (segment (start 159.4 68.6) (end 159.4 67.8) (width 0.6) (layer "B.Cu") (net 1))
 (segment (start 100.6 80.6) (end 100.6 79.8) (width 0.6) (layer "B.Cu") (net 1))
 (segment (start 100.6 55.8) (end 159.4 55.8) (width 0.6) (layer "B.Cu") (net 1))
 (segment (start 100.6 75.8) (end 100.6 75) (width 0.6) (layer "B.Cu") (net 1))
 (segment (start 159.4 63.8) (end 159.4 63) (width 0.6) (layer "B.Cu") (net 1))
 (segment (start 100.6 51.8) (end 100.6 51) (width 0.6) (layer "B.Cu") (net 1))
 (segment (start 159.4 63) (end 100.6 63) (width 0.6) (layer "B.Cu") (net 1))
 (segment (start 100.6 98.2) (end 100.6 97.4) (width 0.6) (layer "B.Cu") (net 1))
 (segment (start 159.4 94.2) (end 159.4 93.4) (width 0.6) (layer "B.Cu") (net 1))
 (segment (start 100.6 79.8) (end 159.4 79.8) (width 0.6) (layer "B.Cu") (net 1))
 (segment (start 159.4 79.8) (end 159.4 79) (width 0.6) (layer "B.Cu") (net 1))
 (segment (start 100.6 74.2) (end 100.6 73.4) (width 0.6) (layer "B.Cu") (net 1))
 (segment (start 158.8 99.8) (end 100.6 99.8) (width 0.6) (layer "B.Cu") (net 1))
 (segment (start 159.4 60.6) (end 159.4 59.8) (width 0.6) (layer "B.Cu") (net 1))
 (segment (start 159.4 50.2) (end 101.2 50.2) (width 0.6) (layer "B.Cu") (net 1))
 (segment (start 100.6 69.4) (end 100.6 68.6) (width 0.6) (layer "B.Cu") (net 1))
 (segment (start 159.4 83.8) (end 100.6 83.8) (width 0.6) (layer "B.Cu") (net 1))
 (segment (start 159.4 95.8) (end 159.4 95) (width 0.6) (layer "B.Cu") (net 1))
 (segment (start 100.6 63.8) (end 159.4 63.8) (width 0.6) (layer "B.Cu") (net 1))
 (segment (start 159.4 51) (end 159.4 50.2) (width 0.6) (layer "B.Cu") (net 1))
 (segment (start 100.6 89.4) (end 159.4 89.4) (width 0.6) (layer "B.Cu") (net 1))
 (segment (start 159.4 77.4) (end 100.6 77.4) (width 0.6) (layer "B.Cu") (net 1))
 (segment (start 100.6 60.6) (end 159.4 60.6) (width 0.6) (layer "B.Cu") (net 1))
 (segment (start 100.6 66.2) (end 100.6 65.4) (width 0.6) (layer "B.Cu") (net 1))
 (segment (start 100.6 88.6) (end 100.6 87.8) (width 0.6) (layer "B.Cu") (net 1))
 (segment (start 159.4 78.2) (end 159.4 77.4) (width 0.6) (layer "B.Cu") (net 1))
 (segment (start 159.4 71.8) (end 159.4 71) (width 0.6) (layer "B.Cu") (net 1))
 (segment (start 159.4 61.4) (end 100.6 61.4) (width 0.6) (layer "B.Cu") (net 1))
 (segment (start 158.8 103.2) (end 158.8 100.6) (width 1.4) (layer "B.Cu") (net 1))
 (segment (start 159.4 71) (end 100.6 71) (width 0.6) (layer "B.Cu") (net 1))
 (segment (start 100.6 93.4) (end 100.6 92.6) (width 0.6) (layer "B.Cu") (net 1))
 (segment (start 159.4 93.4) (end 100.6 93.4) (width 0.6) (layer "B.Cu") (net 1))
 (segment (start 100.6 87) (end 100.6 86.2) (width 0.6) (layer "B.Cu") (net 1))
 (segment (start 159.4 75.8) (end 100.6 75.8) (width 0.6) (layer "B.Cu") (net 1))
 (segment (start 100.6 55) (end 100.6 54.2) (width 0.6) (layer "B.Cu") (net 1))
 (segment (start 159.4 72.6) (end 100.6 72.6) (width 0.6) (layer "B.Cu") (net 1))
 (segment (start 100.6 65.4) (end 159.4 65.4) (width 0.6) (layer "B.Cu") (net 1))
 (segment (start 101.2 46.8) (end 105 43) (width 1.4) (layer "B.Cu") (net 1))
 (segment (start 100.6 71) (end 100.6 70.2) (width 0.6) (layer "B.Cu") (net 1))
 (segment (start 159.4 67.8) (end 100.6 67.8) (width 0.6) (layer "B.Cu") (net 1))
 (segment (start 100.6 73.4) (end 159.4 73.4) (width 0.6) (layer "B.Cu") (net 1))
 (segment (start 100.6 78.2) (end 159.4 78.2) (width 0.6) (layer "B.Cu") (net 1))
 (segment (start 100.6 57.4) (end 159.4 57.4) (width 0.6) (layer "B.Cu") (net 1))
 (segment (start 100.6 94.2) (end 159.4 94.2) (width 0.6) (layer "B.Cu") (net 1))
 (segment (start 100.6 70.2) (end 159.4 70.2) (width 0.6) (layer "B.Cu") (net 1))
 (segment (start 159.4 69.4) (end 100.6 69.4) (width 0.6) (layer "B.Cu") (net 1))
 (segment (start 159.4 70.2) (end 159.4 69.4) (width 0.6) (layer "B.Cu") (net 1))
 (segment (start 100.6 56.6) (end 100.6 55.8) (width 0.6) (layer "B.Cu") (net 1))
 (segment (start 100.6 99) (end 159.4 99) (width 0.6) (layer "B.Cu") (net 1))
 (segment (start 100.6 52.6) (end 159.4 52.6) (width 0.6) (layer "B.Cu") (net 1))
 (segment (start 159.4 57.4) (end 159.4 56.6) (width 0.6) (layer "B.Cu") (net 1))
 (segment (start 100.6 82.2) (end 100.6 81.4) (width 0.6) (layer "B.Cu") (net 1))
 (segment (start 100.6 58.2) (end 100.6 57.4) (width 0.6) (layer "B.Cu") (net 1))
 (segment (start 158.8 103.2) (end 155 107) (width 1.4) (layer "B.Cu") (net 1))
 (segment (start 159.4 74.2) (end 100.6 74.2) (width 0.6) (layer "B.Cu") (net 1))
 (segment (start 159.4 92.6) (end 159.4 91.8) (width 0.6) (layer "B.Cu") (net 1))
 (segment (start 159.4 79) (end 100.6 79) (width 0.6) (layer "B.Cu") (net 1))
 (segment (start 100.6 91.8) (end 100.6 91) (width 0.6) (layer "B.Cu") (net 1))
 (segment (start 100.6 99.8) (end 100.6 99) (width 0.6) (layer "B.Cu") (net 1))
 (segment (start 159.4 96.6) (end 100.6 96.6) (width 0.6) (layer "B.Cu") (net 1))
 (segment (start 100.6 86.2) (end 159.4 86.2) (width 0.6) (layer "B.Cu") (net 1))
 (segment (start 100.6 61.4) (end 100.6 60.6) (width 0.6) (layer "B.Cu") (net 1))
 (segment (start 159.4 62.2) (end 159.4 61.4) (width 0.6) (layer "B.Cu") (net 1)))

